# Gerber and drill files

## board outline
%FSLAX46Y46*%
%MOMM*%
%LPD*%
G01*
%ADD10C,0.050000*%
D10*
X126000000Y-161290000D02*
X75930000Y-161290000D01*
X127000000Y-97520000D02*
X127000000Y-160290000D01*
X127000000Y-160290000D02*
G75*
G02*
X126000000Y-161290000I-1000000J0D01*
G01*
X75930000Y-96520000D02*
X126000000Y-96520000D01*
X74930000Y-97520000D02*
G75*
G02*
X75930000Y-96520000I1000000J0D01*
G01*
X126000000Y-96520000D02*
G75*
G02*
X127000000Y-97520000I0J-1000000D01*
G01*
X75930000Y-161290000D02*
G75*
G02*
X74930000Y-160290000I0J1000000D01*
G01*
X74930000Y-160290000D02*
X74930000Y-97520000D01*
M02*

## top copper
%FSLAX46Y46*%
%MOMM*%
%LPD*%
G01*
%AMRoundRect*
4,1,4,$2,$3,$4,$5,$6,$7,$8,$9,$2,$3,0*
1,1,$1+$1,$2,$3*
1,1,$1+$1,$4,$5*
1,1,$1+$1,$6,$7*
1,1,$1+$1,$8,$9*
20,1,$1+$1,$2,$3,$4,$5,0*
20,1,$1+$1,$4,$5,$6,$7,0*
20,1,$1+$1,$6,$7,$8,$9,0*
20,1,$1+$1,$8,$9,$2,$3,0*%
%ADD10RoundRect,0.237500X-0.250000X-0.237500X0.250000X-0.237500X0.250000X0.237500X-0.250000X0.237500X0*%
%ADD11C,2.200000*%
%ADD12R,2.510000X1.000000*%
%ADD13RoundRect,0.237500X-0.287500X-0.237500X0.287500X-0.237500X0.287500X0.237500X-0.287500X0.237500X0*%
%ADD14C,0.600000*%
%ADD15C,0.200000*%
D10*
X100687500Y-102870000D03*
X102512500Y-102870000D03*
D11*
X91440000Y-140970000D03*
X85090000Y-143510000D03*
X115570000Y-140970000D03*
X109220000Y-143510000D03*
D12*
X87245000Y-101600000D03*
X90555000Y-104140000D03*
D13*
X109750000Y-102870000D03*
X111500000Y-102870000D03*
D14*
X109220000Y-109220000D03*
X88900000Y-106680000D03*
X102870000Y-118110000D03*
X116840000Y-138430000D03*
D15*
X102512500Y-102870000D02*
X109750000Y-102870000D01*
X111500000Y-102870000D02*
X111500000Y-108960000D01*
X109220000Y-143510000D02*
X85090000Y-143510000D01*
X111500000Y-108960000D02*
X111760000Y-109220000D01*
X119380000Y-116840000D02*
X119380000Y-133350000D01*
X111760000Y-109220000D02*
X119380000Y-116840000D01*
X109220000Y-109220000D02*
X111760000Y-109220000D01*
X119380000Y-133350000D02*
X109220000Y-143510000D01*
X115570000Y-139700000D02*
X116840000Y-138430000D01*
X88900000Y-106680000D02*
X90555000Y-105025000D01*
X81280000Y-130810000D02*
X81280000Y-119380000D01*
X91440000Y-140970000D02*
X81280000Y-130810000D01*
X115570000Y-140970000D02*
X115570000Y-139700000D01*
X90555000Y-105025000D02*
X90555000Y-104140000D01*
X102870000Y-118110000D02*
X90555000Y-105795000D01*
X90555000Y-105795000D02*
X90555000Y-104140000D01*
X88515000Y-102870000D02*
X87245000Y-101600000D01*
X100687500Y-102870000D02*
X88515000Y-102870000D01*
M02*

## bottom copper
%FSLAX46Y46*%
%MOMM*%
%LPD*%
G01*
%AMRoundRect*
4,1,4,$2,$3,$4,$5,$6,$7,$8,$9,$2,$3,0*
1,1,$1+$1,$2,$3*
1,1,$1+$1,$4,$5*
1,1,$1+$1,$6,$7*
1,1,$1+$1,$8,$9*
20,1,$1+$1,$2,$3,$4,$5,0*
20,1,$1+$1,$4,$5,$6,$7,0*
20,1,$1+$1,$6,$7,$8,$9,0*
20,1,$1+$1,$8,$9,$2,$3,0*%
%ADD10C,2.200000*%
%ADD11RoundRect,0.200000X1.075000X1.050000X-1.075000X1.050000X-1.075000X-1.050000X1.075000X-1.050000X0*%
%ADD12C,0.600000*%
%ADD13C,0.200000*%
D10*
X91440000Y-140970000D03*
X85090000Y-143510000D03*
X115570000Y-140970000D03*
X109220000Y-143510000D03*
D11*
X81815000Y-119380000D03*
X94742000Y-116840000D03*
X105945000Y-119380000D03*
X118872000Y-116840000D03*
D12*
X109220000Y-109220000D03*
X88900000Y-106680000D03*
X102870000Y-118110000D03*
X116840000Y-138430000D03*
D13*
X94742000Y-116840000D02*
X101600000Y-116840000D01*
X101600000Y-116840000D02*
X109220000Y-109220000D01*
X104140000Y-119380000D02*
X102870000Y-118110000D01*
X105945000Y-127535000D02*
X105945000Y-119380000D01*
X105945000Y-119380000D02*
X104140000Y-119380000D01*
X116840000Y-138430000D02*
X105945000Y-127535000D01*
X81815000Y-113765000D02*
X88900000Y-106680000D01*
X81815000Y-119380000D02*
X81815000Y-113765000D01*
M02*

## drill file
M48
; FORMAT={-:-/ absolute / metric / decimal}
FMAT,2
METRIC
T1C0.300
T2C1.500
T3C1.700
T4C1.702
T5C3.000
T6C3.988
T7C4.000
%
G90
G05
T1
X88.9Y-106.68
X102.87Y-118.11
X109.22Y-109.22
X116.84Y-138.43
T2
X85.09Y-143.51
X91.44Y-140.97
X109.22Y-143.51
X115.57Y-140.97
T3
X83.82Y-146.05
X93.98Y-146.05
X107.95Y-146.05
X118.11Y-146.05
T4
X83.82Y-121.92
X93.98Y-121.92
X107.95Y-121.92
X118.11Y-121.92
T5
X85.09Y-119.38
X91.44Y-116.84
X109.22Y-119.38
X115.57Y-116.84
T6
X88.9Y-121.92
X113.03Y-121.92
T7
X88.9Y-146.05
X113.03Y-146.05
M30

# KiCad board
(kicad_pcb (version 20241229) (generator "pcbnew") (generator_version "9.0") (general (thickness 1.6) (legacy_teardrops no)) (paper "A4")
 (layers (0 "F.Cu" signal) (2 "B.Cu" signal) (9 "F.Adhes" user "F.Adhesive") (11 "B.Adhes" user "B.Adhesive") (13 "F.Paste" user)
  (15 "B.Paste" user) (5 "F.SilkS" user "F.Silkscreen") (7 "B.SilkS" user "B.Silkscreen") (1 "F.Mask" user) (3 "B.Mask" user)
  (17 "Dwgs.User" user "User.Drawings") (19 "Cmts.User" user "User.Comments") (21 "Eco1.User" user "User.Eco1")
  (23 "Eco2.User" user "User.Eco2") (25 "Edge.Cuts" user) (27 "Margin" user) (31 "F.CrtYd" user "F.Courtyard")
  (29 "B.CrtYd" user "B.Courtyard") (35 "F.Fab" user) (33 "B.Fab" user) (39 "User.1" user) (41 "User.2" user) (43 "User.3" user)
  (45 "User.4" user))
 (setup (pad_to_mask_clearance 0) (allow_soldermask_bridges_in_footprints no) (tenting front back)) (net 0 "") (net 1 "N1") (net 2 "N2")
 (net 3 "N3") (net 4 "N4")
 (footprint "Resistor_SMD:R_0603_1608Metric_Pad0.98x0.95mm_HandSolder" (layer "F.Cu") (at 101.6 102.87)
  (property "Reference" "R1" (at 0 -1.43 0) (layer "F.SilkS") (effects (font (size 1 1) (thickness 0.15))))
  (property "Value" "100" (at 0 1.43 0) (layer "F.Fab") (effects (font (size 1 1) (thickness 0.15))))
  (pad "1" smd roundrect (at -0.9125 0) (size 0.975 0.95) (layers "F.Cu" "F.Mask" "F.Paste") (roundrect_rratio 0.25) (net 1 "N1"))
  (pad "2" smd roundrect (at 0.9125 0) (size 0.975 0.95) (layers "F.Cu" "F.Mask" "F.Paste") (roundrect_rratio 0.25) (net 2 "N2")))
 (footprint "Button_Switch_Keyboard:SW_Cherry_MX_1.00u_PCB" (layer "F.Cu") (at 91.44 140.97)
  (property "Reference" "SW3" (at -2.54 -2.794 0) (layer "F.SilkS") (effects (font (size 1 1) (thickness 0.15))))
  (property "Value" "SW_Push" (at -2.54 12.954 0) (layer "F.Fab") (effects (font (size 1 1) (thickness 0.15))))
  (pad "" np_thru_hole circle (at -7.62 5.08) (size 1.7 1.7) (drill 1.7) (layers "*.Cu" "*.Mask"))
  (pad "" np_thru_hole circle (at -2.54 5.08) (size 4 4) (drill 4) (layers "*.Cu" "*.Mask"))
  (pad "" np_thru_hole circle (at 2.54 5.08) (size 1.7 1.7) (drill 1.7) (layers "*.Cu" "*.Mask"))
  (pad "1" thru_hole circle (at 0 0) (size 2.2 2.2) (drill 1.5) (layers "*.Cu" "*.Mask") (remove_unused_layers no) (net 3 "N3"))
  (pad "2" thru_hole circle (at -6.35 2.54) (size 2.2 2.2) (drill 1.5) (layers "*.Cu" "*.Mask") (remove_unused_layers no) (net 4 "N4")))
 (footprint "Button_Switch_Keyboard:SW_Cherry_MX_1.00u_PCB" (layer "F.Cu") (at 115.57 140.97)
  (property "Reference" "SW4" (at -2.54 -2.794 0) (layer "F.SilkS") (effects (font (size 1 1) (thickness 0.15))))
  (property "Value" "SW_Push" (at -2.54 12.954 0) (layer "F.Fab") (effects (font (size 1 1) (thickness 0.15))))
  (pad "" np_thru_hole circle (at -7.62 5.08) (size 1.7 1.7) (drill 1.7) (layers "*.Cu" "*.Mask"))
  (pad "" np_thru_hole circle (at -2.54 5.08) (size 4 4) (drill 4) (layers "*.Cu" "*.Mask"))
  (pad "" np_thru_hole circle (at 2.54 5.08) (size 1.7 1.7) (drill 1.7) (layers "*.Cu" "*.Mask"))
  (pad "1" thru_hole circle (at 0 0) (size 2.2 2.2) (drill 1.5) (layers "*.Cu" "*.Mask") (remove_unused_layers no) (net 3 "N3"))
  (pad "2" thru_hole circle (at -6.35 2.54) (size 2.2 2.2) (drill 1.5) (layers "*.Cu" "*.Mask") (remove_unused_layers no) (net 4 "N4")))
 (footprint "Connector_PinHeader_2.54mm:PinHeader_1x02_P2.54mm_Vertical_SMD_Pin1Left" (layer "F.Cu") (at 88.9 102.87)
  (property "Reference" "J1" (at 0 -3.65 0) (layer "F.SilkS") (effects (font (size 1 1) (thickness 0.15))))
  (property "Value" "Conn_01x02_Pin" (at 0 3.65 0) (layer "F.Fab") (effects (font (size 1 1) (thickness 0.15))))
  (pad "1" smd rect (at -1.655 -1.27) (size 2.51 1) (layers "F.Cu" "F.Mask" "F.Paste") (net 1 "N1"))
  (pad "2" smd rect (at 1.655 1.27) (size 2.51 1) (layers "F.Cu" "F.Mask" "F.Paste") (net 3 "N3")))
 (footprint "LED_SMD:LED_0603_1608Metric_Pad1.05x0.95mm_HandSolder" (layer "F.Cu") (at 110.625 102.87)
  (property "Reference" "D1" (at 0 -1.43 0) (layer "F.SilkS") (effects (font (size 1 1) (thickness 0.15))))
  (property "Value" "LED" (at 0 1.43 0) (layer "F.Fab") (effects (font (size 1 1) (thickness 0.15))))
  (pad "1" smd roundrect (at -0.875 0) (size 1.05 0.95) (layers "F.Cu" "F.Mask" "F.Paste") (roundrect_rratio 0.25) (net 2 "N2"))
  (pad "2" smd roundrect (at 0.875 0) (size 1.05 0.95) (layers "F.Cu" "F.Mask" "F.Paste") (roundrect_rratio 0.25) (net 4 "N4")))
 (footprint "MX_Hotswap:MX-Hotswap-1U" (layer "B.Cu") (at 88.9 121.92 180)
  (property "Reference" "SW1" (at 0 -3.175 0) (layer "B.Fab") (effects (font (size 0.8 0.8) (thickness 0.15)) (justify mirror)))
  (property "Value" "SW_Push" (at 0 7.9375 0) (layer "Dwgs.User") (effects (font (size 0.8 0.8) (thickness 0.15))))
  (pad "" np_thru_hole circle (at -5.08 0 228.099) (size 1.7018 1.7018) (drill 1.7018) (layers "*.Cu" "*.Mask"))
  (pad "" np_thru_hole circle (at -2.54 5.08 180) (size 3 3) (drill 3) (layers "*.Cu" "*.Mask"))
  (pad "" np_thru_hole circle (at 0 0 180) (size 3.9878 3.9878) (drill 3.9878) (layers "*.Cu" "*.Mask"))
  (pad "" np_thru_hole circle (at 3.81 2.54 180) (size 3 3) (drill 3) (layers "*.Cu" "*.Mask"))
  (pad "" np_thru_hole circle (at 5.08 0 228.099) (size 1.7018 1.7018) (drill 1.7018) (layers "*.Cu" "*.Mask"))
  (pad "1" smd roundrect (at 7.085 2.54 180) (size 2.55 2.5) (layers "B.Cu" "B.Mask" "B.Paste") (roundrect_rratio 0.08) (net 3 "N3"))
  (pad "2" smd roundrect (at -5.842 5.08 180) (size 2.55 2.5) (layers "B.Cu" "B.Mask" "B.Paste") (roundrect_rratio 0.08) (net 4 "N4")))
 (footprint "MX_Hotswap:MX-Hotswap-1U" (layer "B.Cu") (at 113.03 121.92 180)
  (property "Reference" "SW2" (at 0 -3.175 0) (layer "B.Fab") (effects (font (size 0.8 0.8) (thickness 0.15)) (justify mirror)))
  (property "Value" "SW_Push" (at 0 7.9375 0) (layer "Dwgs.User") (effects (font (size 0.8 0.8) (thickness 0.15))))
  (pad "" np_thru_hole circle (at -5.08 0 228.099) (size 1.7018 1.7018) (drill 1.7018) (layers "*.Cu" "*.Mask"))
  (pad "" np_thru_hole circle (at -2.54 5.08 180) (size 3 3) (drill 3) (layers "*.Cu" "*.Mask"))
  (pad "" np_thru_hole circle (at 0 0 180) (size 3.9878 3.9878) (drill 3.9878) (layers "*.Cu" "*.Mask"))
  (pad "" np_thru_hole circle (at 3.81 2.54 180) (size 3 3) (drill 3) (layers "*.Cu" "*.Mask"))
  (pad "" np_thru_hole circle (at 5.08 0 228.099) (size 1.7018 1.7018) (drill 1.7018) (layers "*.Cu" "*.Mask"))
  (pad "1" smd roundrect (at 7.085 2.54 180) (size 2.55 2.5) (layers "B.Cu" "B.Mask" "B.Paste") (roundrect_rratio 0.08) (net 3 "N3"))
  (pad "2" smd roundrect (at -5.842 5.08 180) (size 2.55 2.5) (layers "B.Cu" "B.Mask" "B.Paste") (roundrect_rratio 0.08) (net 4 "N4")))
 (gr_line (start 126 161.29) (end 75.93 161.29) (stroke (width 0.05) (type default)) (layer "Edge.Cuts"))
 (gr_line (start 127 97.52) (end 127 160.29) (stroke (width 0.05) (type default)) (layer "Edge.Cuts"))
 (gr_arc (start 127 160.29) (mid 126.707107 160.997107) (end 126 161.29) (stroke (width 0.05) (type default)) (layer "Edge.Cuts"))
 (gr_line (start 75.93 96.52) (end 126 96.52) (stroke (width 0.05) (type default)) (layer "Edge.Cuts"))
 (gr_arc (start 74.93 97.52) (mid 75.222893 96.812893) (end 75.93 96.52) (stroke (width 0.05) (type default)) (layer "Edge.Cuts"))
 (gr_arc (start 126 96.52) (mid 126.707107 96.812893) (end 127 97.52) (stroke (width 0.05) (type default)) (layer "Edge.Cuts"))
 (gr_arc (start 75.93 161.29) (mid 75.222893 160.997107) (end 74.93 160.29) (stroke (width 0.05) (type default)) (layer "Edge.Cuts"))
 (gr_line (start 74.93 160.29) (end 74.93 97.52) (stroke (width 0.05) (type default)) (layer "Edge.Cuts"))
 (segment (start 102.5125 102.87) (end 109.75 102.87) (width 0.2) (layer "F.Cu") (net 2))
 (segment (start 111.5 102.87) (end 111.5 108.96) (width 0.2) (layer "F.Cu") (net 4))
 (segment (start 109.22 143.51) (end 85.09 143.51) (width 0.2) (layer "F.Cu") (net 4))
 (segment (start 111.5 108.96) (end 111.76 109.22) (width 0.2) (layer "F.Cu") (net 4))
 (segment (start 119.38 116.84) (end 119.38 133.35) (width 0.2) (layer "F.Cu") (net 4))
 (segment (start 111.76 109.22) (end 119.38 116.84) (width 0.2) (layer "F.Cu") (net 4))
 (segment (start 109.22 109.22) (end 111.76 109.22) (width 0.2) (layer "F.Cu") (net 4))
 (segment (start 119.38 133.35) (end 109.22 143.51) (width 0.2) (layer "F.Cu") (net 4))
 (via (at 109.22 109.22) (size 0.6) (drill 0.3) (layers "F.Cu" "B.Cu") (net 4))
 (segment (start 94.742 116.84) (end 101.6 116.84) (width 0.2) (layer "B.Cu") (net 4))
 (segment (start 101.6 116.84) (end 109.22 109.22) (width 0.2) (layer "B.Cu") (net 4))
 (segment (start 115.57 139.7) (end 116.84 138.43) (width 0.2) (layer "F.Cu") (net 3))
 (segment (start 88.9 106.68) (end 90.555 105.025) (width 0.2) (layer "F.Cu") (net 3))
 (segment (start 81.28 130.81) (end 81.28 119.38) (width 0.2) (layer "F.Cu") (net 3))
 (segment (start 91.44 140.97) (end 81.28 130.81) (width 0.2) (layer "F.Cu") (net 3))
 (segment (start 115.57 140.97) (end 115.57 139.7) (width 0.2) (layer "F.Cu") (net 3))
 (segment (start 90.555 105.025) (end 90.555 104.14) (width 0.2) (layer "F.Cu") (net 3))
 (segment (start 102.87 118.11) (end 90.555 105.795) (width 0.2) (layer "F.Cu") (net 3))
 (segment (start 90.555 105.795) (end 90.555 104.14) (width 0.2) (layer "F.Cu") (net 3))
 (via (at 88.9 106.68) (size 0.6) (drill 0.3) (layers "F.Cu" "B.Cu") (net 3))
 (via (at 102.87 118.11) (size 0.6) (drill 0.3) (layers "F.Cu" "B.Cu") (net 3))
 (via (at 116.84 138.43) (size 0.6) (drill 0.3) (layers "F.Cu" "B.Cu") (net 3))
 (segment (start 104.14 119.38) (end 102.87 118.11) (width 0.2) (layer "B.Cu") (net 3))
 (segment (start 105.945 127.535) (end 105.945 119.38) (width 0.2) (layer "B.Cu") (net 3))
 (segment (start 105.945 119.38) (end 104.14 119.38) (width 0.2) (layer "B.Cu") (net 3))
 (segment (start 116.84 138.43) (end 105.945 127.535) (width 0.2) (layer "B.Cu") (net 3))
 (segment (start 81.815 113.765) (end 88.9 106.68) (width 0.2) (layer "B.Cu") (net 3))
 (segment (start 81.815 119.38) (end 81.815 113.765) (width 0.2) (layer "B.Cu") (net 3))
 (segment (start 88.515 102.87) (end 87.245 101.6) (width 0.2) (layer "F.Cu") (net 1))
 (segment (start 100.6875 102.87) (end 88.515 102.87) (width 0.2) (layer "F.Cu") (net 1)))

